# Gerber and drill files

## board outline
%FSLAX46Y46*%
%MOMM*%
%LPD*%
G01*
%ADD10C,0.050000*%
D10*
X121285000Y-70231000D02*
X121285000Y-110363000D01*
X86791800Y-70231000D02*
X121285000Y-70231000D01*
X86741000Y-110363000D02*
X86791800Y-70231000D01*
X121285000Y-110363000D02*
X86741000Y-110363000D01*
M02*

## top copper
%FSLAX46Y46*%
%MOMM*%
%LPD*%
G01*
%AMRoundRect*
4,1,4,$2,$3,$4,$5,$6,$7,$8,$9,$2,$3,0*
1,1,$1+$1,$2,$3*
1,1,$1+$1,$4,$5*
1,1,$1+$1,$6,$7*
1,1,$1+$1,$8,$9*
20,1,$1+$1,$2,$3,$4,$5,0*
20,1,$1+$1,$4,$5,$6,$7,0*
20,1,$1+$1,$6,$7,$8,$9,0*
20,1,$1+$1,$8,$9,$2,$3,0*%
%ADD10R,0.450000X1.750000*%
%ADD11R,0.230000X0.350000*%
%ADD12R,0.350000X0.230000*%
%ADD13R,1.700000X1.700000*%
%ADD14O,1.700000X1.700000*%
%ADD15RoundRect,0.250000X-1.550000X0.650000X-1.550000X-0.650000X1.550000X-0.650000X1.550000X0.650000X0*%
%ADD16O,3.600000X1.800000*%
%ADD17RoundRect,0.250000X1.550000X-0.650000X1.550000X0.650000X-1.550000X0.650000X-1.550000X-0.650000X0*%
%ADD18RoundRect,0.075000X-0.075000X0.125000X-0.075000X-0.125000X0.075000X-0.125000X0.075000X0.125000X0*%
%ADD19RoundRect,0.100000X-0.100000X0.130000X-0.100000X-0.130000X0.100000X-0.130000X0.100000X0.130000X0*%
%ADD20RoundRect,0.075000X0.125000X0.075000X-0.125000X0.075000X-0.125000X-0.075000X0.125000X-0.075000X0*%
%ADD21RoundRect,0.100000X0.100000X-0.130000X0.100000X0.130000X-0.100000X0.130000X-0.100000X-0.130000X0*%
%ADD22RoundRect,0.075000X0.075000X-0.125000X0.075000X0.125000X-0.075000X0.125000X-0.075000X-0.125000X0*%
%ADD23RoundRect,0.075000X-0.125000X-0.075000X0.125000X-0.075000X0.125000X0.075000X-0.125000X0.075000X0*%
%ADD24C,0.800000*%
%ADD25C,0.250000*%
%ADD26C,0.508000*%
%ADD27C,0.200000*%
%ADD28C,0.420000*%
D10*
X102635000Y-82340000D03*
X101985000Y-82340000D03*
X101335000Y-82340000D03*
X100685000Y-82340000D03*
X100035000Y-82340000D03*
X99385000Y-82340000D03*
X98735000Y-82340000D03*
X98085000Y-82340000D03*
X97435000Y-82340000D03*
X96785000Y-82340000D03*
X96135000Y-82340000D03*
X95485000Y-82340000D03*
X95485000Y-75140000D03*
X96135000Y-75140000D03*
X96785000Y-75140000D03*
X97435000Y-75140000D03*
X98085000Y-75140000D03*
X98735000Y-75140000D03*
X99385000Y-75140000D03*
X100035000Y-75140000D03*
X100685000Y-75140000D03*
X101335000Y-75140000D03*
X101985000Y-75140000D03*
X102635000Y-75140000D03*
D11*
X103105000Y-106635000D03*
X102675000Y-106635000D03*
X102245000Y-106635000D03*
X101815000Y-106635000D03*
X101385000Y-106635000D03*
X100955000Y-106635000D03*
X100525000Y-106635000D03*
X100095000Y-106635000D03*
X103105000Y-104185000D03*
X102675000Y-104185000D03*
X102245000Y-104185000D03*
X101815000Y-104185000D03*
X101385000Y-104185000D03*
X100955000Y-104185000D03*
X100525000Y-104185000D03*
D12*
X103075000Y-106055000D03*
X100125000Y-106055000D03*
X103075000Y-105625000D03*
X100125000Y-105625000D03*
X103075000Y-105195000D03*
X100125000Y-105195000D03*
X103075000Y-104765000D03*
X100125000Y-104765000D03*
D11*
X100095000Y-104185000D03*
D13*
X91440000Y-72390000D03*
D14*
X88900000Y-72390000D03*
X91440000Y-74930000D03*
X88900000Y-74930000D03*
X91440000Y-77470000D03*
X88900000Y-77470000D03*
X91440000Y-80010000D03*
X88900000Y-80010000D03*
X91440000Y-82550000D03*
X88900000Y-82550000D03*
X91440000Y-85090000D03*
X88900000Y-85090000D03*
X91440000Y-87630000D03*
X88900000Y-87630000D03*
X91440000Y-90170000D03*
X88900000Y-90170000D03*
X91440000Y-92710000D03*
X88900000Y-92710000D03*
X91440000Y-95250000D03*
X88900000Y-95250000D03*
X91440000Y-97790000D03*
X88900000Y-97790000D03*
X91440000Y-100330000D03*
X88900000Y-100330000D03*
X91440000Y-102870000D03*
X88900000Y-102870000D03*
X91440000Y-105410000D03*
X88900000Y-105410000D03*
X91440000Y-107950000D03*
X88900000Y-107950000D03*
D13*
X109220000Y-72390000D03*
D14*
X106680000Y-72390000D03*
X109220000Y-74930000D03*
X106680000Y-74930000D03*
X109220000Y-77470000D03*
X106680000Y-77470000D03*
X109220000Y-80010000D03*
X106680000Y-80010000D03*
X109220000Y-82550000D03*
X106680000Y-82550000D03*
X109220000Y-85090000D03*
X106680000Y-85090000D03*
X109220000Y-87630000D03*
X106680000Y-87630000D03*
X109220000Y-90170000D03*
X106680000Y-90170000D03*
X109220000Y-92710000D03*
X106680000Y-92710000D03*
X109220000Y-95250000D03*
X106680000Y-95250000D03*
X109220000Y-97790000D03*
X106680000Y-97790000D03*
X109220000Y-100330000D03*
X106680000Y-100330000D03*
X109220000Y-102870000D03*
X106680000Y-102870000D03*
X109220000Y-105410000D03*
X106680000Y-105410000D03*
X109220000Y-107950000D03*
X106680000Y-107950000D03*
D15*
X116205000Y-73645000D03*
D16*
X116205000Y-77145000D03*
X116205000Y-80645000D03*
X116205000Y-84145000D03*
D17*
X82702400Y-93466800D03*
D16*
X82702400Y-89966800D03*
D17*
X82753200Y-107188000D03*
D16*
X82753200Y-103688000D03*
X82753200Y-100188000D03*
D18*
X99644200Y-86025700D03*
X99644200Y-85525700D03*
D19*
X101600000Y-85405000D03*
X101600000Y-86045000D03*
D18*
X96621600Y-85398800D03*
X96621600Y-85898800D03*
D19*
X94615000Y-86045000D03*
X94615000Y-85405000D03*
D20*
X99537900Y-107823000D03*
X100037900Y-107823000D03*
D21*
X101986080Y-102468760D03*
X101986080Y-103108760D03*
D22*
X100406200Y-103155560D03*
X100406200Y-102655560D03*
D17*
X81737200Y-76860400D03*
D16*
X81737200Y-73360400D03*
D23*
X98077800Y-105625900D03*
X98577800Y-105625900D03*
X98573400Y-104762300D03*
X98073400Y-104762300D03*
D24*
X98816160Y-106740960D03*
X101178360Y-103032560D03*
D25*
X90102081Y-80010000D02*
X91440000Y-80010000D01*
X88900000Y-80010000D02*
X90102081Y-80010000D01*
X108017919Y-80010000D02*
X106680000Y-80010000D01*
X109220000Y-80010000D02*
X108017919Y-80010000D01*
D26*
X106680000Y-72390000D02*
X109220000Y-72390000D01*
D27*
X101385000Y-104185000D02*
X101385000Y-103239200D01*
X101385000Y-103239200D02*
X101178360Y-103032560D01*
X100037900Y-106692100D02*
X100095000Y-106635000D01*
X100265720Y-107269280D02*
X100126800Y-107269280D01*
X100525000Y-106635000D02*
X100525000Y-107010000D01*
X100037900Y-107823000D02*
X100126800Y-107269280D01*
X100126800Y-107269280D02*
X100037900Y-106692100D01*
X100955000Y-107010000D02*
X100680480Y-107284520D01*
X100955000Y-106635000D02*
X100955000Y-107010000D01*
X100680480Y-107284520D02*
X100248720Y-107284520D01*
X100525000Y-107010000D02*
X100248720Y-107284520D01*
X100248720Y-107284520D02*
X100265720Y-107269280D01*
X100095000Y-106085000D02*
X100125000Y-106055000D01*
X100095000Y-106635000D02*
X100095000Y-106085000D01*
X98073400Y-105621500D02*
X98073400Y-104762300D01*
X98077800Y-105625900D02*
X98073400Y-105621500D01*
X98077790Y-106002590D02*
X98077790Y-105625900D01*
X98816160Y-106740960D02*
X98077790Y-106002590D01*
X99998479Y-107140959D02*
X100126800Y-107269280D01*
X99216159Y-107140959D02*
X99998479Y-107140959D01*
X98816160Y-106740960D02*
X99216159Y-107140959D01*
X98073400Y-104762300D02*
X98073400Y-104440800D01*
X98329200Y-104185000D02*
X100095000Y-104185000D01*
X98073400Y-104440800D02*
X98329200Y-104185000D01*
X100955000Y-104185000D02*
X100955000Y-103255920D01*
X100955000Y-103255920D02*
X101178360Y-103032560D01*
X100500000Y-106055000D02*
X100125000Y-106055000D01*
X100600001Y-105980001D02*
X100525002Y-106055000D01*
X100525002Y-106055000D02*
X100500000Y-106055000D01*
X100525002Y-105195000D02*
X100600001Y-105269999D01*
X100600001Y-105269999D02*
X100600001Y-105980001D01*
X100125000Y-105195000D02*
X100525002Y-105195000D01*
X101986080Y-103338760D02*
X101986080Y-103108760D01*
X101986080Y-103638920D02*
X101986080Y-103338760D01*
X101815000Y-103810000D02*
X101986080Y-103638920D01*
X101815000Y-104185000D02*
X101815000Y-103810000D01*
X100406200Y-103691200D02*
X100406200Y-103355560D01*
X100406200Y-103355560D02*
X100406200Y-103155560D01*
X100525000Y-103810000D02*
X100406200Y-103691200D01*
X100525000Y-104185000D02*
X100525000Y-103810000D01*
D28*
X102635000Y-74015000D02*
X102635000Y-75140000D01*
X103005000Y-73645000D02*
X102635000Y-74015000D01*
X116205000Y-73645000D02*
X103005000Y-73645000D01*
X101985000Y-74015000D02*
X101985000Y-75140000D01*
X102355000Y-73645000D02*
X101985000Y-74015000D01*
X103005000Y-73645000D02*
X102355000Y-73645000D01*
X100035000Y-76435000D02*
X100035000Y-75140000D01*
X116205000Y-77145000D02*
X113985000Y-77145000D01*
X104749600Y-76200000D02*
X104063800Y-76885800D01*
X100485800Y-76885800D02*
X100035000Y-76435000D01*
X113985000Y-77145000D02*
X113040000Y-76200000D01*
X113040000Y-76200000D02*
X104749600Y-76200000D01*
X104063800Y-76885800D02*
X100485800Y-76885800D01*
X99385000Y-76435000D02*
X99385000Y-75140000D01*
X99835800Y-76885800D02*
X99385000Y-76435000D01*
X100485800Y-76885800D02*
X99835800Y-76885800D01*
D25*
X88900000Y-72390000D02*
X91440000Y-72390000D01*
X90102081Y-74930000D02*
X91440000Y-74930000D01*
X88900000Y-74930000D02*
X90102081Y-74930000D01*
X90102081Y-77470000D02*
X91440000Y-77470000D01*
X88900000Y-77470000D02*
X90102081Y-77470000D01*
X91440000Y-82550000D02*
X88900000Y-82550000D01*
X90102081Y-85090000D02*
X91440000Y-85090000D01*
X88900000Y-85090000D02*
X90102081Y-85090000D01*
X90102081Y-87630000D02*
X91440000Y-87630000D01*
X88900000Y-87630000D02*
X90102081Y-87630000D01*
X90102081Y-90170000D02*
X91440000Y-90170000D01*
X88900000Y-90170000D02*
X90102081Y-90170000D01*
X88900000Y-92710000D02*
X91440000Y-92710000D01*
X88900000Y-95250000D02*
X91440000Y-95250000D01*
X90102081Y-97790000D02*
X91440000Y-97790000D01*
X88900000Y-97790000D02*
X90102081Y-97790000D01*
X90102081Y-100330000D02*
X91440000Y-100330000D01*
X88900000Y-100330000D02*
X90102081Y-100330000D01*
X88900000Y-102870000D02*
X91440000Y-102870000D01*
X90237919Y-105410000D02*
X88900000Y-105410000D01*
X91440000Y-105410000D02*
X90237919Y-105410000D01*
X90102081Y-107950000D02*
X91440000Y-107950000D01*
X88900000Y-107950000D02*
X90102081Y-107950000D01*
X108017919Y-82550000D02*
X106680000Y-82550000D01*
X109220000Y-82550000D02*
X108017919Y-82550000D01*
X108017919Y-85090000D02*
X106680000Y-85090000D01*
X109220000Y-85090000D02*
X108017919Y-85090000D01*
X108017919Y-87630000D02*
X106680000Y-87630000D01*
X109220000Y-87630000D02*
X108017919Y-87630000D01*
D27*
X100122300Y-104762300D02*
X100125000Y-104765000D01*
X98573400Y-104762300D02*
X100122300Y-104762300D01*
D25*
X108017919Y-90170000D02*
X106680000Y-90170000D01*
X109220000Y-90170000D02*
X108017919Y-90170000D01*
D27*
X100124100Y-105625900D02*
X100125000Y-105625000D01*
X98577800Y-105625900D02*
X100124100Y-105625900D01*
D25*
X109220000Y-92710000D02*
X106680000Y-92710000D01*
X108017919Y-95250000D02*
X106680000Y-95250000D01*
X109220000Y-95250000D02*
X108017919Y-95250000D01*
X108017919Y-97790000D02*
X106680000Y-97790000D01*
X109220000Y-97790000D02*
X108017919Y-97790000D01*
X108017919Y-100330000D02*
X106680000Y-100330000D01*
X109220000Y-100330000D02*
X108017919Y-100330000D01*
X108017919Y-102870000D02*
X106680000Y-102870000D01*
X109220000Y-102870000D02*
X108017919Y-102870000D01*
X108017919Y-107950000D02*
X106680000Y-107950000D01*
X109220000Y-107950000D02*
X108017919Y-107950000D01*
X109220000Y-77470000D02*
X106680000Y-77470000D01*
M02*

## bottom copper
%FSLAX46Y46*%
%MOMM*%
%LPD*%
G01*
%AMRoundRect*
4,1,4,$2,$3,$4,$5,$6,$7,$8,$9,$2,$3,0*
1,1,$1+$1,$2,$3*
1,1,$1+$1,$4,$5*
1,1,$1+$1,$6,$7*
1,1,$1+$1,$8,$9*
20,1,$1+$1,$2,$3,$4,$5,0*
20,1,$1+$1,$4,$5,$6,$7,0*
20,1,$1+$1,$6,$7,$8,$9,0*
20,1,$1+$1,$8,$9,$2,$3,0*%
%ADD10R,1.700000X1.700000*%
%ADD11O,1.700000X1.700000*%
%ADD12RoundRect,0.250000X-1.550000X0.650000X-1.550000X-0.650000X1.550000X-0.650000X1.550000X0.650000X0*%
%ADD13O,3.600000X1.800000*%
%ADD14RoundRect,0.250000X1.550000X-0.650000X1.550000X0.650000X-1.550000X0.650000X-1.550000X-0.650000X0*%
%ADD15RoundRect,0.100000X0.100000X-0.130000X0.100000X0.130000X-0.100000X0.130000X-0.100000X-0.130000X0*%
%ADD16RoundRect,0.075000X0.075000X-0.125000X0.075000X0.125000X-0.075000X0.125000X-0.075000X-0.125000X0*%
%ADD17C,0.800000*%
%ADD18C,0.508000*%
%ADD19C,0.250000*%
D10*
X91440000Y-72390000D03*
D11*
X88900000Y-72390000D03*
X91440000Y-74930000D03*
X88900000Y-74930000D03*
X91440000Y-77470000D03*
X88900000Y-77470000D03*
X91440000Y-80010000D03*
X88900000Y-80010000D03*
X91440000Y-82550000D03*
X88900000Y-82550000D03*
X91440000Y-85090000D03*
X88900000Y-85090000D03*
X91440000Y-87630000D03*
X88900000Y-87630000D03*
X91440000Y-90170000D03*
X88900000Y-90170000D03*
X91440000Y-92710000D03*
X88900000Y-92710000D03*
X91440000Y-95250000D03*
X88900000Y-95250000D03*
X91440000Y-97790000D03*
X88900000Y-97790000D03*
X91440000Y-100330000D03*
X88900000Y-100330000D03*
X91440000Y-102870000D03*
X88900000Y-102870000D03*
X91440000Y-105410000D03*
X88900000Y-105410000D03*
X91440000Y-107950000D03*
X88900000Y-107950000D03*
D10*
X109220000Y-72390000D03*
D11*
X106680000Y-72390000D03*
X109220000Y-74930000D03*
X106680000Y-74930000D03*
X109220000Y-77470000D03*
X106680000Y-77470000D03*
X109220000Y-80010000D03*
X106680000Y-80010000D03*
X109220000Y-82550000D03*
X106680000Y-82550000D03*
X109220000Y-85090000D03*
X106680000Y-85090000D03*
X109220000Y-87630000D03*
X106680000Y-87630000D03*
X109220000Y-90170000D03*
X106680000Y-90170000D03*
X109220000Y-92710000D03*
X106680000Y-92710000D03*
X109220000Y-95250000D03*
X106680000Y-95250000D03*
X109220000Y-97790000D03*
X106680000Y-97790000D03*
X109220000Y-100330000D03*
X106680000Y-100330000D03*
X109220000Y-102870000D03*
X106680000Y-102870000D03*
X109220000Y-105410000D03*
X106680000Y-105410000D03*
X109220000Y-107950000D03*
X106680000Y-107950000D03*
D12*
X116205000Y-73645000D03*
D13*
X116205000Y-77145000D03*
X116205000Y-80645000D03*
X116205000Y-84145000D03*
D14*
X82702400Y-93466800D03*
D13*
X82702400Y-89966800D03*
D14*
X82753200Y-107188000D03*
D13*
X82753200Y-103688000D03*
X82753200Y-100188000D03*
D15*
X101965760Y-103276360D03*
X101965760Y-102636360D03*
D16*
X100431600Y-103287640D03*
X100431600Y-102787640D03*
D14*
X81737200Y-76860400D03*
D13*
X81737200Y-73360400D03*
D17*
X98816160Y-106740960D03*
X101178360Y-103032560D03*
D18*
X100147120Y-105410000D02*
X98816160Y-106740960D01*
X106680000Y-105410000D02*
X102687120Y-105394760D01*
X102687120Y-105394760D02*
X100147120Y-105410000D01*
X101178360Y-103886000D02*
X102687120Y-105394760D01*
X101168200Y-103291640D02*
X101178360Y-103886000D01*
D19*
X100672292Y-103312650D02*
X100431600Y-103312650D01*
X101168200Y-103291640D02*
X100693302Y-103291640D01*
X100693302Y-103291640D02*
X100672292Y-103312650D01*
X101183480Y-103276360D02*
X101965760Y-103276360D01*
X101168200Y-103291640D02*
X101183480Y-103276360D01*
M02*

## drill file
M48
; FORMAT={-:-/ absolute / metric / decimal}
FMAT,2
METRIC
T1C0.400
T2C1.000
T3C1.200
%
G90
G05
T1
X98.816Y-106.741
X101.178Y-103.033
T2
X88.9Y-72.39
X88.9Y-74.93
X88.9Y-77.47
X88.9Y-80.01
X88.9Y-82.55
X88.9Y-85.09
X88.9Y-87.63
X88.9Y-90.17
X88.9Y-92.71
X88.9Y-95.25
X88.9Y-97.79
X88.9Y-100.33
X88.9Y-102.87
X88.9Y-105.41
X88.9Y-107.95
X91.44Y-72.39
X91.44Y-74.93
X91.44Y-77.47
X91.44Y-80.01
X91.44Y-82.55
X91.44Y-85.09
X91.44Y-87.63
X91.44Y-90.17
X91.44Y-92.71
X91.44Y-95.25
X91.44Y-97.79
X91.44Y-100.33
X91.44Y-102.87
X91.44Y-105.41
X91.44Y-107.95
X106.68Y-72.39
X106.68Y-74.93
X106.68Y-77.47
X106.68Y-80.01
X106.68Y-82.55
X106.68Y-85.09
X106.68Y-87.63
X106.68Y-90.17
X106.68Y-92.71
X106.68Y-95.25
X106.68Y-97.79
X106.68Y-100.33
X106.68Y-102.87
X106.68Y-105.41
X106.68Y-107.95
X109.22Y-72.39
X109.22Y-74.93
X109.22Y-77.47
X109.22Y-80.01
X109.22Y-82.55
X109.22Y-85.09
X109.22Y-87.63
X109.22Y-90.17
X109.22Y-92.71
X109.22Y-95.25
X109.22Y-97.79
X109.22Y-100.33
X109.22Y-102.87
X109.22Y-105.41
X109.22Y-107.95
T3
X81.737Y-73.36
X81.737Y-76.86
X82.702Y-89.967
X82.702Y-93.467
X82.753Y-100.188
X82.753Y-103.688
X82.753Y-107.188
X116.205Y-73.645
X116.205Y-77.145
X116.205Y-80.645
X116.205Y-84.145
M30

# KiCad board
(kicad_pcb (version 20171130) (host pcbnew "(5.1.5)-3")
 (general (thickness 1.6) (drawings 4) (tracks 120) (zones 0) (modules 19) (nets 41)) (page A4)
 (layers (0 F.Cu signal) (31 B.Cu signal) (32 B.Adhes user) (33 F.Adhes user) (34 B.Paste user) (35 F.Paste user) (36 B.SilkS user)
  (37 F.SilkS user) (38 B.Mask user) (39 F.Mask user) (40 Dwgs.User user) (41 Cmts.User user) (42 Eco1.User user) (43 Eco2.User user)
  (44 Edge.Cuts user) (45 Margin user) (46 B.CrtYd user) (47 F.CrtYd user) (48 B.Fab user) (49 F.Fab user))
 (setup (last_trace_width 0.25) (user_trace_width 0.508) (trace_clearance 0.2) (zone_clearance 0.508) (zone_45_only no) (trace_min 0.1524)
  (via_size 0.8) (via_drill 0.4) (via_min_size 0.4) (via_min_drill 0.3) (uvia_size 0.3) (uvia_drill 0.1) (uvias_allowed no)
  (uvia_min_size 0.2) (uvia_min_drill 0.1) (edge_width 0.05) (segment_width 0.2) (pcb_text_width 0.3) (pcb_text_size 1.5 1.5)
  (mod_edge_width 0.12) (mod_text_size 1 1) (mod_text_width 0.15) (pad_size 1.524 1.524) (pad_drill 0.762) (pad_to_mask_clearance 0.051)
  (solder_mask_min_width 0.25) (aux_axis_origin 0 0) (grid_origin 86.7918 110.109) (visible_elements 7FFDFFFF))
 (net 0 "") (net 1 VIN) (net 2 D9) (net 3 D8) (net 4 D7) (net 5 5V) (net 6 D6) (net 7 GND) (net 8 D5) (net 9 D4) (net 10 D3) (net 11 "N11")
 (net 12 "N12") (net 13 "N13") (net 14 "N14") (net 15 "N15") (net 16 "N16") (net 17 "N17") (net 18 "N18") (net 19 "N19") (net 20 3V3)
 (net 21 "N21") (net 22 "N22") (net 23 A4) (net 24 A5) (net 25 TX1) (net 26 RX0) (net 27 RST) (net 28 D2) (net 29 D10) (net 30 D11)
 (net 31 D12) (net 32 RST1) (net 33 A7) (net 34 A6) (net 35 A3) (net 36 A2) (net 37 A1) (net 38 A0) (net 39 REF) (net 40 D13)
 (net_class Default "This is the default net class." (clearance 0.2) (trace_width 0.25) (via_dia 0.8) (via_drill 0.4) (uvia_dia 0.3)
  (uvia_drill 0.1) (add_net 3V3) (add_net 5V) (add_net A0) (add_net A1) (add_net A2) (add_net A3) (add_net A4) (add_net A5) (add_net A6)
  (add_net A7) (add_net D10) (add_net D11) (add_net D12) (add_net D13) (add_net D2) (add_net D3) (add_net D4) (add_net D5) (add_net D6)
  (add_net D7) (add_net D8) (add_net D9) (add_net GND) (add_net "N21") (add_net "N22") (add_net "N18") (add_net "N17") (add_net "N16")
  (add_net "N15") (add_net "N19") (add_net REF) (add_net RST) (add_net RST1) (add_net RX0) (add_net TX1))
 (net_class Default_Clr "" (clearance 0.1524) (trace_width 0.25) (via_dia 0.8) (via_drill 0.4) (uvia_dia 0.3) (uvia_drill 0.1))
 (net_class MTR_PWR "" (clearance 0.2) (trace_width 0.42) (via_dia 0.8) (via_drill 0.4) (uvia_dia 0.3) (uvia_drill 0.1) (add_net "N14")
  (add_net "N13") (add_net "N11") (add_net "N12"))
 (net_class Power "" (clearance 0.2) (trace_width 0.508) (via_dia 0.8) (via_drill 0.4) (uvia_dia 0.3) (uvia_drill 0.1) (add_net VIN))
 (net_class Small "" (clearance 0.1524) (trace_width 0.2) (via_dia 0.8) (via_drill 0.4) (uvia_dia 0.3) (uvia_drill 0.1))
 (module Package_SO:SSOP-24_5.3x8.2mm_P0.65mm (layer F.Cu) (at 99.06 78.74 270)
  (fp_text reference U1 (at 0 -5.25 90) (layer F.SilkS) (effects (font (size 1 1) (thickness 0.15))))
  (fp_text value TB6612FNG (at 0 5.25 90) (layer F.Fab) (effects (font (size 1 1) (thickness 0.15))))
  (pad 24 smd rect (at 3.6 -3.575 270) (size 1.75 0.45) (layers F.Cu F.Paste F.Mask) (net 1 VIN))
  (pad 23 smd rect (at 3.6 -2.925 270) (size 1.75 0.45) (layers F.Cu F.Paste F.Mask) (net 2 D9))
  (pad 22 smd rect (at 3.6 -2.275 270) (size 1.75 0.45) (layers F.Cu F.Paste F.Mask) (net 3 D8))
  (pad 21 smd rect (at 3.6 -1.625 270) (size 1.75 0.45) (layers F.Cu F.Paste F.Mask) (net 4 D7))
  (pad 20 smd rect (at 3.6 -0.975 270) (size 1.75 0.45) (layers F.Cu F.Paste F.Mask) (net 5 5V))
  (pad 19 smd rect (at 3.6 -0.325 270) (size 1.75 0.45) (layers F.Cu F.Paste F.Mask) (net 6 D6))
  (pad 18 smd rect (at 3.6 0.325 270) (size 1.75 0.45) (layers F.Cu F.Paste F.Mask) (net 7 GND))
  (pad 17 smd rect (at 3.6 0.975 270) (size 1.75 0.45) (layers F.Cu F.Paste F.Mask) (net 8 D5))
  (pad 16 smd rect (at 3.6 1.625 270) (size 1.75 0.45) (layers F.Cu F.Paste F.Mask) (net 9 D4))
  (pad 15 smd rect (at 3.6 2.275 270) (size 1.75 0.45) (layers F.Cu F.Paste F.Mask) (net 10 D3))
  (pad 14 smd rect (at 3.6 2.925 270) (size 1.75 0.45) (layers F.Cu F.Paste F.Mask) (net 1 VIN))
  (pad 13 smd rect (at 3.6 3.575 270) (size 1.75 0.45) (layers F.Cu F.Paste F.Mask) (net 1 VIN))
  (pad 12 smd rect (at -3.6 3.575 270) (size 1.75 0.45) (layers F.Cu F.Paste F.Mask) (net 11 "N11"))
  (pad 11 smd rect (at -3.6 2.925 270) (size 1.75 0.45) (layers F.Cu F.Paste F.Mask) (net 11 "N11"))
  (pad 10 smd rect (at -3.6 2.275 270) (size 1.75 0.45) (layers F.Cu F.Paste F.Mask) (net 7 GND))
  (pad 9 smd rect (at -3.6 1.625 270) (size 1.75 0.45) (layers F.Cu F.Paste F.Mask) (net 7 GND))
  (pad 8 smd rect (at -3.6 0.975 270) (size 1.75 0.45) (layers F.Cu F.Paste F.Mask) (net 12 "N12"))
  (pad 7 smd rect (at -3.6 0.325 270) (size 1.75 0.45) (layers F.Cu F.Paste F.Mask) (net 12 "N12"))
  (pad 6 smd rect (at -3.6 -0.325 270) (size 1.75 0.45) (layers F.Cu F.Paste F.Mask) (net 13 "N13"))
  (pad 5 smd rect (at -3.6 -0.975 270) (size 1.75 0.45) (layers F.Cu F.Paste F.Mask) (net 13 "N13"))
  (pad 4 smd rect (at -3.6 -1.625 270) (size 1.75 0.45) (layers F.Cu F.Paste F.Mask) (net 7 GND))
  (pad 3 smd rect (at -3.6 -2.275 270) (size 1.75 0.45) (layers F.Cu F.Paste F.Mask) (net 7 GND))
  (pad 2 smd rect (at -3.6 -2.925 270) (size 1.75 0.45) (layers F.Cu F.Paste F.Mask) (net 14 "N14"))
  (pad 1 smd rect (at -3.6 -3.575 270) (size 1.75 0.45) (layers F.Cu F.Paste F.Mask) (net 14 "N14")))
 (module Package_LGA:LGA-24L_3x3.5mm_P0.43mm (layer F.Cu) (at 101.6 105.41)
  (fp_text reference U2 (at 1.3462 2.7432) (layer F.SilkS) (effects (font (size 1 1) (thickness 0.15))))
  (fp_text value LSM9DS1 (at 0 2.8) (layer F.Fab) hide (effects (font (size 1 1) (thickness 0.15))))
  (pad 13 smd rect (at 1.505 1.225) (size 0.23 0.35) (layers F.Cu F.Paste F.Mask) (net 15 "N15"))
  (pad 12 smd rect (at 1.075 1.225) (size 0.23 0.35) (layers F.Cu F.Paste F.Mask) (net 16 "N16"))
  (pad 11 smd rect (at 0.645 1.225) (size 0.23 0.35) (layers F.Cu F.Paste F.Mask) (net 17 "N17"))
  (pad 10 smd rect (at 0.215 1.225) (size 0.23 0.35) (layers F.Cu F.Paste F.Mask) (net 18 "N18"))
  (pad 9 smd rect (at -0.215 1.225) (size 0.23 0.35) (layers F.Cu F.Paste F.Mask) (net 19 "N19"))
  (pad 8 smd rect (at -0.645 1.225) (size 0.23 0.35) (layers F.Cu F.Paste F.Mask) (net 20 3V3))
  (pad 7 smd rect (at -1.075 1.225) (size 0.23 0.35) (layers F.Cu F.Paste F.Mask) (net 20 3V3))
  (pad 6 smd rect (at -1.505 1.225) (size 0.23 0.35) (layers F.Cu F.Paste F.Mask) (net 20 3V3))
  (pad 18 smd rect (at 1.505 -1.225) (size 0.23 0.35) (layers F.Cu F.Paste F.Mask) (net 7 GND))
  (pad 19 smd rect (at 1.075 -1.225) (size 0.23 0.35) (layers F.Cu F.Paste F.Mask) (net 7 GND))
  (pad 20 smd rect (at 0.645 -1.225) (size 0.23 0.35) (layers F.Cu F.Paste F.Mask) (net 7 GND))
  (pad 21 smd rect (at 0.215 -1.225) (size 0.23 0.35) (layers F.Cu F.Paste F.Mask) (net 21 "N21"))
  (pad 22 smd rect (at -0.215 -1.225) (size 0.23 0.35) (layers F.Cu F.Paste F.Mask) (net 20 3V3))
  (pad 23 smd rect (at -0.645 -1.225) (size 0.23 0.35) (layers F.Cu F.Paste F.Mask) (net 20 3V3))
  (pad 24 smd rect (at -1.075 -1.225) (size 0.23 0.35) (layers F.Cu F.Paste F.Mask) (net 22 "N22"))
  (pad 14 smd rect (at 1.475 0.645) (size 0.35 0.23) (layers F.Cu F.Paste F.Mask) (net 7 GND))
  (pad 5 smd rect (at -1.475 0.645) (size 0.35 0.23) (layers F.Cu F.Paste F.Mask) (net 20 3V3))
  (pad 15 smd rect (at 1.475 0.215) (size 0.35 0.23) (layers F.Cu F.Paste F.Mask) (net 7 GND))
  (pad 4 smd rect (at -1.475 0.215) (size 0.35 0.23) (layers F.Cu F.Paste F.Mask) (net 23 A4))
  (pad 16 smd rect (at 1.475 -0.215) (size 0.35 0.23) (layers F.Cu F.Paste F.Mask) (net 7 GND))
  (pad 3 smd rect (at -1.475 -0.215) (size 0.35 0.23) (layers F.Cu F.Paste F.Mask) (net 20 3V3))
  (pad 17 smd rect (at 1.475 -0.645) (size 0.35 0.23) (layers F.Cu F.Paste F.Mask) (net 7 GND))
  (pad 2 smd rect (at -1.475 -0.645) (size 0.35 0.23) (layers F.Cu F.Paste F.Mask) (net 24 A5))
  (pad 1 smd rect (at -1.505 -1.225) (size 0.23 0.35) (layers F.Cu F.Paste F.Mask) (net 20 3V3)))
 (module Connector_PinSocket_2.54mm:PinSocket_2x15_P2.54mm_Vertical (layer F.Cu) (at 91.44 72.39)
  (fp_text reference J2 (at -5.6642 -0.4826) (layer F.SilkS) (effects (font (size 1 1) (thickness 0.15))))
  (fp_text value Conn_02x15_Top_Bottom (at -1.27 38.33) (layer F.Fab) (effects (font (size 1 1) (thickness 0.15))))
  (pad 1 thru_hole rect (at 0 0) (size 1.7 1.7) (drill 1) (layers *.Cu *.Mask) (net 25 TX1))
  (pad 2 thru_hole oval (at -2.54 0) (size 1.7 1.7) (drill 1) (layers *.Cu *.Mask) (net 25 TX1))
  (pad 3 thru_hole oval (at 0 2.54) (size 1.7 1.7) (drill 1) (layers *.Cu *.Mask) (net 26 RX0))
  (pad 4 thru_hole oval (at -2.54 2.54) (size 1.7 1.7) (drill 1) (layers *.Cu *.Mask) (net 26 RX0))
  (pad 5 thru_hole oval (at 0 5.08) (size 1.7 1.7) (drill 1) (layers *.Cu *.Mask) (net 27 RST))
  (pad 6 thru_hole oval (at -2.54 5.08) (size 1.7 1.7) (drill 1) (layers *.Cu *.Mask) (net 27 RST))
  (pad 7 thru_hole oval (at 0 7.62) (size 1.7 1.7) (drill 1) (layers *.Cu *.Mask) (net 7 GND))
  (pad 8 thru_hole oval (at -2.54 7.62) (size 1.7 1.7) (drill 1) (layers *.Cu *.Mask) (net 7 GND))
  (pad 9 thru_hole oval (at 0 10.16) (size 1.7 1.7) (drill 1) (layers *.Cu *.Mask) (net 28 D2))
  (pad 10 thru_hole oval (at -2.54 10.16) (size 1.7 1.7) (drill 1) (layers *.Cu *.Mask) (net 28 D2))
  (pad 11 thru_hole oval (at 0 12.7) (size 1.7 1.7) (drill 1) (layers *.Cu *.Mask) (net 10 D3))
  (pad 12 thru_hole oval (at -2.54 12.7) (size 1.7 1.7) (drill 1) (layers *.Cu *.Mask) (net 10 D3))
  (pad 13 thru_hole oval (at 0 15.24) (size 1.7 1.7) (drill 1) (layers *.Cu *.Mask) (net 9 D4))
  (pad 14 thru_hole oval (at -2.54 15.24) (size 1.7 1.7) (drill 1) (layers *.Cu *.Mask) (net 9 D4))
  (pad 15 thru_hole oval (at 0 17.78) (size 1.7 1.7) (drill 1) (layers *.Cu *.Mask) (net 8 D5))
  (pad 16 thru_hole oval (at -2.54 17.78) (size 1.7 1.7) (drill 1) (layers *.Cu *.Mask) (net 8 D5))
  (pad 17 thru_hole oval (at 0 20.32) (size 1.7 1.7) (drill 1) (layers *.Cu *.Mask) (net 6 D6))
  (pad 18 thru_hole oval (at -2.54 20.32) (size 1.7 1.7) (drill 1) (layers *.Cu *.Mask) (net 6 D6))
  (pad 19 thru_hole oval (at 0 22.86) (size 1.7 1.7) (drill 1) (layers *.Cu *.Mask) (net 4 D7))
  (pad 20 thru_hole oval (at -2.54 22.86) (size 1.7 1.7) (drill 1) (layers *.Cu *.Mask) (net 4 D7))
  (pad 21 thru_hole oval (at 0 25.4) (size 1.7 1.7) (drill 1) (layers *.Cu *.Mask) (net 3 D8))
  (pad 22 thru_hole oval (at -2.54 25.4) (size 1.7 1.7) (drill 1) (layers *.Cu *.Mask) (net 3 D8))
  (pad 23 thru_hole oval (at 0 27.94) (size 1.7 1.7) (drill 1) (layers *.Cu *.Mask) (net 2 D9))
  (pad 24 thru_hole oval (at -2.54 27.94) (size 1.7 1.7) (drill 1) (layers *.Cu *.Mask) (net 2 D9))
  (pad 25 thru_hole oval (at 0 30.48) (size 1.7 1.7) (drill 1) (layers *.Cu *.Mask) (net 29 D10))
  (pad 26 thru_hole oval (at -2.54 30.48) (size 1.7 1.7) (drill 1) (layers *.Cu *.Mask) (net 29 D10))
  (pad 27 thru_hole oval (at 0 33.02) (size 1.7 1.7) (drill 1) (layers *.Cu *.Mask) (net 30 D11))
  (pad 28 thru_hole oval (at -2.54 33.02) (size 1.7 1.7) (drill 1) (layers *.Cu *.Mask) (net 30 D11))
  (pad 29 thru_hole oval (at 0 35.56) (size 1.7 1.7) (drill 1) (layers *.Cu *.Mask) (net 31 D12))
  (pad 30 thru_hole oval (at -2.54 35.56) (size 1.7 1.7) (drill 1) (layers *.Cu *.Mask) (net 31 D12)))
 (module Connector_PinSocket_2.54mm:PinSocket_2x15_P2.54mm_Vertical (layer F.Cu) (at 109.22 72.39)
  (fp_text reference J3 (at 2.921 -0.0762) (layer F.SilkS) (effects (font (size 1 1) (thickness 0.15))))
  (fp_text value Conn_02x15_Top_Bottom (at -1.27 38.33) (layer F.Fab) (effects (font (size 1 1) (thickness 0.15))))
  (pad 1 thru_hole rect (at 0 0) (size 1.7 1.7) (drill 1) (layers *.Cu *.Mask) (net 1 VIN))
  (pad 2 thru_hole oval (at -2.54 0) (size 1.7 1.7) (drill 1) (layers *.Cu *.Mask) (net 1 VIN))
  (pad 3 thru_hole oval (at 0 2.54) (size 1.7 1.7) (drill 1) (layers *.Cu *.Mask) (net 7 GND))
  (pad 4 thru_hole oval (at -2.54 2.54) (size 1.7 1.7) (drill 1) (layers *.Cu *.Mask) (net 7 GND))
  (pad 5 thru_hole oval (at 0 5.08) (size 1.7 1.7) (drill 1) (layers *.Cu *.Mask) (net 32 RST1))
  (pad 6 thru_hole oval (at -2.54 5.08) (size 1.7 1.7) (drill 1) (layers *.Cu *.Mask) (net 32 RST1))
  (pad 7 thru_hole oval (at 0 7.62) (size 1.7 1.7) (drill 1) (layers *.Cu *.Mask) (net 5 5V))
  (pad 8 thru_hole oval (at -2.54 7.62) (size 1.7 1.7) (drill 1) (layers *.Cu *.Mask) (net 5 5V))
  (pad 9 thru_hole oval (at 0 10.16) (size 1.7 1.7) (drill 1) (layers *.Cu *.Mask) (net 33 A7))
  (pad 10 thru_hole oval (at -2.54 10.16) (size 1.7 1.7) (drill 1) (layers *.Cu *.Mask) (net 33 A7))
  (pad 11 thru_hole oval (at 0 12.7) (size 1.7 1.7) (drill 1) (layers *.Cu *.Mask) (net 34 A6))
  (pad 12 thru_hole oval (at -2.54 12.7) (size 1.7 1.7) (drill 1) (layers *.Cu *.Mask) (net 34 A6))
  (pad 13 thru_hole oval (at 0 15.24) (size 1.7 1.7) (drill 1) (layers *.Cu *.Mask) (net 24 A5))
  (pad 14 thru_hole oval (at -2.54 15.24) (size 1.7 1.7) (drill 1) (layers *.Cu *.Mask) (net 24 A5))
  (pad 15 thru_hole oval (at 0 17.78) (size 1.7 1.7) (drill 1) (layers *.Cu *.Mask) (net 23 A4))
  (pad 16 thru_hole oval (at -2.54 17.78) (size 1.7 1.7) (drill 1) (layers *.Cu *.Mask) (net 23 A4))
  (pad 17 thru_hole oval (at 0 20.32) (size 1.7 1.7) (drill 1) (layers *.Cu *.Mask) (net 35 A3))
  (pad 18 thru_hole oval (at -2.54 20.32) (size 1.7 1.7) (drill 1) (layers *.Cu *.Mask) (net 35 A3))
  (pad 19 thru_hole oval (at 0 22.86) (size 1.7 1.7) (drill 1) (layers *.Cu *.Mask) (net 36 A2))
  (pad 20 thru_hole oval (at -2.54 22.86) (size 1.7 1.7) (drill 1) (layers *.Cu *.Mask) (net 36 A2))
  (pad 21 thru_hole oval (at 0 25.4) (size 1.7 1.7) (drill 1) (layers *.Cu *.Mask) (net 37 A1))
  (pad 22 thru_hole oval (at -2.54 25.4) (size 1.7 1.7) (drill 1) (layers *.Cu *.Mask) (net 37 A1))
  (pad 23 thru_hole oval (at 0 27.94) (size 1.7 1.7) (drill 1) (layers *.Cu *.Mask) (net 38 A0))
  (pad 24 thru_hole oval (at -2.54 27.94) (size 1.7 1.7) (drill 1) (layers *.Cu *.Mask) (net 38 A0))
  (pad 25 thru_hole oval (at 0 30.48) (size 1.7 1.7) (drill 1) (layers *.Cu *.Mask) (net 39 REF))
  (pad 26 thru_hole oval (at -2.54 30.48) (size 1.7 1.7) (drill 1) (layers *.Cu *.Mask) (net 39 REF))
  (pad 27 thru_hole oval (at 0 33.02) (size 1.7 1.7) (drill 1) (layers *.Cu *.Mask) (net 20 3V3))
  (pad 28 thru_hole oval (at -2.54 33.02) (size 1.7 1.7) (drill 1) (layers *.Cu *.Mask) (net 20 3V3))
  (pad 29 thru_hole oval (at 0 35.56) (size 1.7 1.7) (drill 1) (layers *.Cu *.Mask) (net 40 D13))
  (pad 30 thru_hole oval (at -2.54 35.56) (size 1.7 1.7) (drill 1) (layers *.Cu *.Mask) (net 40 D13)))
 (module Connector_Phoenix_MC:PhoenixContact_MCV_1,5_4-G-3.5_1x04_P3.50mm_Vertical (layer F.Cu) (at 116.205 73.645 270)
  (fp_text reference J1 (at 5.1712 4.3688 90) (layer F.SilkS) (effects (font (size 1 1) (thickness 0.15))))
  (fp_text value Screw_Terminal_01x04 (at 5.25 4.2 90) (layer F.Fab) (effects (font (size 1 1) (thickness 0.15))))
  (pad 1 thru_hole roundrect (at 0 0 270) (size 1.8 3.6) (drill 1.2) (layers *.Cu *.Mask) (roundrect_rratio 0.138889) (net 14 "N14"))
  (pad 2 thru_hole oval (at 3.5 0 270) (size 1.8 3.6) (drill 1.2) (layers *.Cu *.Mask) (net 13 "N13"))
  (pad 3 thru_hole oval (at 7 0 270) (size 1.8 3.6) (drill 1.2) (layers *.Cu *.Mask) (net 11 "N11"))
  (pad 4 thru_hole oval (at 10.5 0 270) (size 1.8 3.6) (drill 1.2) (layers *.Cu *.Mask) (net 12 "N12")))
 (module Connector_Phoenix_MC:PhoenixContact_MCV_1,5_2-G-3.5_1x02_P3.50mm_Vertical (layer F.Cu) (at 82.7024 93.4668 90)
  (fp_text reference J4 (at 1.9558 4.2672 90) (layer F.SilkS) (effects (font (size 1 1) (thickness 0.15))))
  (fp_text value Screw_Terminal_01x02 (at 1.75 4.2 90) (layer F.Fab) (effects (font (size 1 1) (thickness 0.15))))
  (pad 1 thru_hole roundrect (at 0 0 90) (size 1.8 3.6) (drill 1.2) (layers *.Cu *.Mask) (roundrect_rratio 0.138889) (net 1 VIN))
  (pad 2 thru_hole oval (at 3.5 0 90) (size 1.8 3.6) (drill 1.2) (layers *.Cu *.Mask) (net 7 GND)))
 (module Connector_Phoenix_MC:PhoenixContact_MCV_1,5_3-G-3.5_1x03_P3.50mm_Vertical (layer F.Cu) (at 82.7532 107.188 90)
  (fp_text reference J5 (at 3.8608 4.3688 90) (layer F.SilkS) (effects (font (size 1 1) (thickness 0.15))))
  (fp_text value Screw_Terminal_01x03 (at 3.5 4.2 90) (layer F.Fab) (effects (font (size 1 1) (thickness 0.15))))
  (pad 1 thru_hole roundrect (at 0 0 90) (size 1.8 3.6) (drill 1.2) (layers *.Cu *.Mask) (roundrect_rratio 0.138889) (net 29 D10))
  (pad 2 thru_hole oval (at 3.5 0 90) (size 1.8 3.6) (drill 1.2) (layers *.Cu *.Mask) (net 30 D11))
  (pad 3 thru_hole oval (at 7 0 90) (size 1.8 3.6) (drill 1.2) (layers *.Cu *.Mask) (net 31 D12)))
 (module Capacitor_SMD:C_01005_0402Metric (layer F.Cu) (at 99.6442 85.7757 270)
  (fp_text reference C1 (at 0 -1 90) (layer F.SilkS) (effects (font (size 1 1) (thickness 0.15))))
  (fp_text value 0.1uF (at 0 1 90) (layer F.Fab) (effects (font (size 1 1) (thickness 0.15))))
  (pad 2 smd roundrect (at 0.25 0 270) (size 0.4 0.3) (layers F.Cu F.Mask) (roundrect_rratio 0.25) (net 7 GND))
  (pad 1 smd roundrect (at -0.25 0 270) (size 0.4 0.3) (layers F.Cu F.Mask) (roundrect_rratio 0.25) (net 5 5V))
  (pad "" smd roundrect (at 0.275 0 270) (size 0.27 0.27) (layers F.Paste) (roundrect_rratio 0.25))
  (pad "" smd roundrect (at -0.275 0 270) (size 0.27 0.27) (layers F.Paste) (roundrect_rratio 0.25)))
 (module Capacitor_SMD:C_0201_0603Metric (layer F.Cu) (at 101.6 85.725 270)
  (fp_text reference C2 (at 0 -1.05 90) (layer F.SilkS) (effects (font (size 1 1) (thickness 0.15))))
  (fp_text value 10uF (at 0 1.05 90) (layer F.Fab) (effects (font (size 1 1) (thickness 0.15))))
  (pad "" smd roundrect (at -0.345 0 270) (size 0.318 0.36) (layers F.Paste) (roundrect_rratio 0.25))
  (pad "" smd roundrect (at 0.345 0 270) (size 0.318 0.36) (layers F.Paste) (roundrect_rratio 0.25))
  (pad 1 smd roundrect (at -0.32 0 270) (size 0.46 0.4) (layers F.Cu F.Mask) (roundrect_rratio 0.25) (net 5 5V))
  (pad 2 smd roundrect (at 0.32 0 270) (size 0.46 0.4) (layers F.Cu F.Mask) (roundrect_rratio 0.25) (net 7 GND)))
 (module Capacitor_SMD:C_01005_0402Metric (layer F.Cu) (at 96.6216 85.6488 270)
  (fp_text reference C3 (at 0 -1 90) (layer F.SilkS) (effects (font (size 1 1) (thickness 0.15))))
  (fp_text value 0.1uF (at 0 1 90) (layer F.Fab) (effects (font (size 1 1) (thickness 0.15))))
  (pad "" smd roundrect (at -0.275 0 270) (size 0.27 0.27) (layers F.Paste) (roundrect_rratio 0.25))
  (pad "" smd roundrect (at 0.275 0 270) (size 0.27 0.27) (layers F.Paste) (roundrect_rratio 0.25))
  (pad 1 smd roundrect (at -0.25 0 270) (size 0.4 0.3) (layers F.Cu F.Mask) (roundrect_rratio 0.25) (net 1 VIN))
  (pad 2 smd roundrect (at 0.25 0 270) (size 0.4 0.3) (layers F.Cu F.Mask) (roundrect_rratio 0.25) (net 7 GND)))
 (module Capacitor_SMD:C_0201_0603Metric (layer F.Cu) (at 94.615 85.725 270)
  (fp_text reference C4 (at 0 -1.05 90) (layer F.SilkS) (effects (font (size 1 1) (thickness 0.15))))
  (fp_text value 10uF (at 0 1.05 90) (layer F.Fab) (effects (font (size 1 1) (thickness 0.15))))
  (pad 2 smd roundrect (at 0.32 0 270) (size 0.46 0.4) (layers F.Cu F.Mask) (roundrect_rratio 0.25) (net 7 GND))
  (pad 1 smd roundrect (at -0.32 0 270) (size 0.46 0.4) (layers F.Cu F.Mask) (roundrect_rratio 0.25) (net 1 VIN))
  (pad "" smd roundrect (at 0.345 0 270) (size 0.318 0.36) (layers F.Paste) (roundrect_rratio 0.25))
  (pad "" smd roundrect (at -0.345 0 270) (size 0.318 0.36) (layers F.Paste) (roundrect_rratio 0.25)))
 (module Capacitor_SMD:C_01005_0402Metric (layer F.Cu) (at 99.7879 107.823 180)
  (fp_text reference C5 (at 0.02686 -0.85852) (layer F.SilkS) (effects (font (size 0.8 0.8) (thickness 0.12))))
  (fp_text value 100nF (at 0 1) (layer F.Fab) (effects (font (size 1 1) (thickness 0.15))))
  (pad 2 smd roundrect (at 0.25 0 180) (size 0.4 0.3) (layers F.Cu F.Mask) (roundrect_rratio 0.25) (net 7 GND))
  (pad 1 smd roundrect (at -0.25 0 180) (size 0.4 0.3) (layers F.Cu F.Mask) (roundrect_rratio 0.25) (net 20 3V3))
  (pad "" smd roundrect (at 0.275 0 180) (size 0.27 0.27) (layers F.Paste) (roundrect_rratio 0.25))
  (pad "" smd roundrect (at -0.275 0 180) (size 0.27 0.27) (layers F.Paste) (roundrect_rratio 0.25)))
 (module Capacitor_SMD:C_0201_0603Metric (layer B.Cu) (at 101.96576 102.95636 90)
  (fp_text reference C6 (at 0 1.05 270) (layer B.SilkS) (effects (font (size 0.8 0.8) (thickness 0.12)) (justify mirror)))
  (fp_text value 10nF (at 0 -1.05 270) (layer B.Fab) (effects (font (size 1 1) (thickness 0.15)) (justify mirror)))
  (pad "" smd roundrect (at -0.345 0 90) (size 0.318 0.36) (layers B.Paste) (roundrect_rratio 0.25))
  (pad "" smd roundrect (at 0.345 0 90) (size 0.318 0.36) (layers B.Paste) (roundrect_rratio 0.25))
  (pad 1 smd roundrect (at -0.32 0 90) (size 0.46 0.4) (layers B.Cu B.Mask) (roundrect_rratio 0.25) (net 20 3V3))
  (pad 2 smd roundrect (at 0.32 0 90) (size 0.46 0.4) (layers B.Cu B.Mask) (roundrect_rratio 0.25) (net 7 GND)))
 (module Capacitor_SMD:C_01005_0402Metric (layer B.Cu) (at 100.4316 103.03764 90)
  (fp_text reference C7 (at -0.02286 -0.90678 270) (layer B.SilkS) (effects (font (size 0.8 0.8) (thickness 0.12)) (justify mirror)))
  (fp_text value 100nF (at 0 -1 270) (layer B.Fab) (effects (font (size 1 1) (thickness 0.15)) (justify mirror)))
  (pad "" smd roundrect (at -0.275 0 90) (size 0.27 0.27) (layers B.Paste) (roundrect_rratio 0.25))
  (pad "" smd roundrect (at 0.275 0 90) (size 0.27 0.27) (layers B.Paste) (roundrect_rratio 0.25))
  (pad 1 smd roundrect (at -0.25 0 90) (size 0.4 0.3) (layers B.Cu B.Mask) (roundrect_rratio 0.25) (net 20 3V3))
  (pad 2 smd roundrect (at 0.25 0 90) (size 0.4 0.3) (layers B.Cu B.Mask) (roundrect_rratio 0.25) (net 7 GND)))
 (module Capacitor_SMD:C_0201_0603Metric (layer F.Cu) (at 101.98608 102.78876 90)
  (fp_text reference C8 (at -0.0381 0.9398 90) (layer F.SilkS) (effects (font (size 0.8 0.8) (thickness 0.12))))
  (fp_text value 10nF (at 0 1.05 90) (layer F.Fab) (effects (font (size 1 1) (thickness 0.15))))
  (pad 2 smd roundrect (at 0.32 0 90) (size 0.46 0.4) (layers F.Cu F.Mask) (roundrect_rratio 0.25) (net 7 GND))
  (pad 1 smd roundrect (at -0.32 0 90) (size 0.46 0.4) (layers F.Cu F.Mask) (roundrect_rratio 0.25) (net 21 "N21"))
  (pad "" smd roundrect (at 0.345 0 90) (size 0.318 0.36) (layers F.Paste) (roundrect_rratio 0.25))
  (pad "" smd roundrect (at -0.345 0 90) (size 0.318 0.36) (layers F.Paste) (roundrect_rratio 0.25)))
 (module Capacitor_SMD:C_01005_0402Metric (layer F.Cu) (at 100.4062 102.90556 90)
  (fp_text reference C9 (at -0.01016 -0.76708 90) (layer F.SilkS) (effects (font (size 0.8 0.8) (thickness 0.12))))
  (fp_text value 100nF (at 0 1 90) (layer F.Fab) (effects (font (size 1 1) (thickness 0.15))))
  (pad "" smd roundrect (at -0.275 0 90) (size 0.27 0.27) (layers F.Paste) (roundrect_rratio 0.25))
  (pad "" smd roundrect (at 0.275 0 90) (size 0.27 0.27) (layers F.Paste) (roundrect_rratio 0.25))
  (pad 1 smd roundrect (at -0.25 0 90) (size 0.4 0.3) (layers F.Cu F.Mask) (roundrect_rratio 0.25) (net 22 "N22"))
  (pad 2 smd roundrect (at 0.25 0 90) (size 0.4 0.3) (layers F.Cu F.Mask) (roundrect_rratio 0.25) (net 7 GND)))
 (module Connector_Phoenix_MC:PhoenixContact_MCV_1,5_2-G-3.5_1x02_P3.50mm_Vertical (layer F.Cu) (at 81.7372 76.8604 90)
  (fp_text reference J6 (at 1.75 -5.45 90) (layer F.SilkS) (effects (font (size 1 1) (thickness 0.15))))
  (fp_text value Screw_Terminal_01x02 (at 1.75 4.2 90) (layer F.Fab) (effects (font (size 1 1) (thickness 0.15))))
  (pad 1 thru_hole roundrect (at 0 0 90) (size 1.8 3.6) (drill 1.2) (layers *.Cu *.Mask) (roundrect_rratio 0.138889) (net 5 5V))
  (pad 2 thru_hole oval (at 3.5 0 90) (size 1.8 3.6) (drill 1.2) (layers *.Cu *.Mask) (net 7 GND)))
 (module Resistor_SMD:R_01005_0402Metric (layer F.Cu) (at 98.3278 105.6259)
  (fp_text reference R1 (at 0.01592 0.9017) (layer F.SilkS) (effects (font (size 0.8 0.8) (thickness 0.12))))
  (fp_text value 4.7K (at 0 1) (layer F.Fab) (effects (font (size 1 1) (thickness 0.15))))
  (pad "" smd roundrect (at -0.275 0) (size 0.27 0.27) (layers F.Paste) (roundrect_rratio 0.25))
  (pad "" smd roundrect (at 0.275 0) (size 0.27 0.27) (layers F.Paste) (roundrect_rratio 0.25))
  (pad 1 smd roundrect (at -0.25 0) (size 0.4 0.3) (layers F.Cu F.Mask) (roundrect_rratio 0.25) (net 20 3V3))
  (pad 2 smd roundrect (at 0.25 0) (size 0.4 0.3) (layers F.Cu F.Mask) (roundrect_rratio 0.25) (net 23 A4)))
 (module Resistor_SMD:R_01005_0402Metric (layer F.Cu) (at 98.3234 104.7623)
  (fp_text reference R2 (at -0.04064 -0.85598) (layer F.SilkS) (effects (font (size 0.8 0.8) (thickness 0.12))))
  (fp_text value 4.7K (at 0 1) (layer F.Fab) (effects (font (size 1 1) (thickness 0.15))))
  (pad 2 smd roundrect (at 0.25 0) (size 0.4 0.3) (layers F.Cu F.Mask) (roundrect_rratio 0.25) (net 24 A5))
  (pad 1 smd roundrect (at -0.25 0) (size 0.4 0.3) (layers F.Cu F.Mask) (roundrect_rratio 0.25) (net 20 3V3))
  (pad "" smd roundrect (at 0.275 0) (size 0.27 0.27) (layers F.Paste) (roundrect_rratio 0.25))
  (pad "" smd roundrect (at -0.275 0) (size 0.27 0.27) (layers F.Paste) (roundrect_rratio 0.25)))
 (gr_line (start 121.285 70.231) (end 121.285 110.363) (layer Edge.Cuts) (width 0.05))
 (gr_line (start 86.7918 70.231) (end 121.285 70.231) (layer Edge.Cuts) (width 0.05))
 (gr_line (start 86.741 110.363) (end 86.7918 70.231) (layer Edge.Cuts) (width 0.05))
 (gr_line (start 121.285 110.363) (end 86.741 110.363) (layer Edge.Cuts) (width 0.05))
 (segment (start 90.102081 80.01) (end 91.44 80.01) (width 0.25) (layer F.Cu) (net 7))
 (segment (start 88.9 80.01) (end 90.102081 80.01) (width 0.25) (layer F.Cu) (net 7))
 (segment (start 108.017919 80.01) (end 106.68 80.01) (width 0.25) (layer F.Cu) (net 5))
 (segment (start 109.22 80.01) (end 108.017919 80.01) (width 0.25) (layer F.Cu) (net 5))
 (segment (start 106.68 72.39) (end 109.22 72.39) (width 0.508) (layer F.Cu) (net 1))
 (segment (start 101.385 104.185) (end 101.385 103.2392) (width 0.2) (layer F.Cu) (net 20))
 (segment (start 101.385 103.2392) (end 101.17836 103.03256) (width 0.2) (layer F.Cu) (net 20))
 (segment (start 100.0379 106.6921) (end 100.095 106.635) (width 0.2) (layer F.Cu) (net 20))
 (segment (start 100.26572 107.26928) (end 100.1268 107.26928) (width 0.2) (layer F.Cu) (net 20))
 (segment (start 100.525 106.635) (end 100.525 107.01) (width 0.2) (layer F.Cu) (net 20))
 (segment (start 100.0379 107.823) (end 100.1268 107.26928) (width 0.2) (layer F.Cu) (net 20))
 (segment (start 100.1268 107.26928) (end 100.0379 106.6921) (width 0.2) (layer F.Cu) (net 20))
 (segment (start 100.955 107.01) (end 100.68048 107.28452) (width 0.2) (layer F.Cu) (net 20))
 (segment (start 100.955 106.635) (end 100.955 107.01) (width 0.2) (layer F.Cu) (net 20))
 (segment (start 100.68048 107.28452) (end 100.24872 107.28452) (width 0.2) (layer F.Cu) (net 20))
 (segment (start 100.525 107.01) (end 100.24872 107.28452) (width 0.2) (layer F.Cu) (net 20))
 (segment (start 100.24872 107.28452) (end 100.26572 107.26928) (width 0.2) (layer F.Cu) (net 20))
 (segment (start 100.095 106.085) (end 100.125 106.055) (width 0.2) (layer F.Cu) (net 20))
 (segment (start 100.095 106.635) (end 100.095 106.085) (width 0.2) (layer F.Cu) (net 20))
 (segment (start 98.0734 105.6215) (end 98.0734 104.7623) (width 0.2) (layer F.Cu) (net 20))
 (segment (start 98.0778 105.6259) (end 98.0734 105.6215) (width 0.2) (layer F.Cu) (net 20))
 (via (at 98.81616 106.74096) (size 0.8) (drill 0.4) (layers F.Cu B.Cu) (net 20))
 (segment (start 100.14712 105.41) (end 98.81616 106.74096) (width 0.508) (layer B.Cu) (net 20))
 (segment (start 98.07779 106.00259) (end 98.07779 105.6259) (width 0.2) (layer F.Cu) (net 20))
 (segment (start 98.81616 106.74096) (end 98.07779 106.00259) (width 0.2) (layer F.Cu) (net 20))
 (segment (start 99.998479 107.140959) (end 100.1268 107.26928) (width 0.2) (layer F.Cu) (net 20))
 (segment (start 99.216159 107.140959) (end 99.998479 107.140959) (width 0.2) (layer F.Cu) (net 20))
 (segment (start 98.81616 106.74096) (end 99.216159 107.140959) (width 0.2) (layer F.Cu) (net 20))
 (segment (start 106.68 105.41) (end 102.68712 105.39476) (width 0.508) (layer B.Cu) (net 20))
 (segment (start 102.68712 105.39476) (end 100.14712 105.41) (width 0.508) (layer B.Cu) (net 20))
 (segment (start 98.0734 104.7623) (end 98.0734 104.4408) (width 0.2) (layer F.Cu) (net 20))
 (segment (start 98.3292 104.185) (end 100.095 104.185) (width 0.2) (layer F.Cu) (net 20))
 (segment (start 98.0734 104.4408) (end 98.3292 104.185) (width 0.2) (layer F.Cu) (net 20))
 (segment (start 101.17836 103.886) (end 102.68712 105.39476) (width 0.508) (layer B.Cu) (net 20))
 (segment (start 101.1682 103.29164) (end 101.17836 103.886) (width 0.508) (layer B.Cu) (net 20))
 (segment (start 100.672292 103.31265) (end 100.4316 103.31265) (width 0.25) (layer B.Cu) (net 20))
 (segment (start 101.1682 103.29164) (end 100.693302 103.29164) (width 0.25) (layer B.Cu) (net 20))
 (segment (start 100.693302 103.29164) (end 100.672292 103.31265) (width 0.25) (layer B.Cu) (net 20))
 (segment (start 101.18348 103.27636) (end 101.96576 103.27636) (width 0.25) (layer B.Cu) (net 20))
 (segment (start 101.1682 103.29164) (end 101.18348 103.27636) (width 0.25) (layer B.Cu) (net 20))
 (via (at 101.17836 103.03256) (size 0.8) (drill 0.4) (layers F.Cu B.Cu) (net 20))
 (segment (start 100.955 104.185) (end 100.955 103.25592) (width 0.2) (layer F.Cu) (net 20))
 (segment (start 100.955 103.25592) (end 101.17836 103.03256) (width 0.2) (layer F.Cu) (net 20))
 (segment (start 100.5 106.055) (end 100.125 106.055) (width 0.2) (layer F.Cu) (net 20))
 (segment (start 100.600001 105.980001) (end 100.525002 106.055) (width 0.2) (layer F.Cu) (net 20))
 (segment (start 100.525002 106.055) (end 100.5 106.055) (width 0.2) (layer F.Cu) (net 20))
 (segment (start 100.525002 105.195) (end 100.600001 105.269999) (width 0.2) (layer F.Cu) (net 20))
 (segment (start 100.600001 105.269999) (end 100.600001 105.980001) (width 0.2) (layer F.Cu) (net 20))
 (segment (start 100.125 105.195) (end 100.525002 105.195) (width 0.2) (layer F.Cu) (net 20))
 (segment (start 101.98608 103.33876) (end 101.98608 103.10876) (width 0.2) (layer F.Cu) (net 21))
 (segment (start 101.98608 103.63892) (end 101.98608 103.33876) (width 0.2) (layer F.Cu) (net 21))
 (segment (start 101.815 103.81) (end 101.98608 103.63892) (width 0.2) (layer F.Cu) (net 21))
 (segment (start 101.815 104.185) (end 101.815 103.81) (width 0.2) (layer F.Cu) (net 21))
 (segment (start 100.4062 103.6912) (end 100.4062 103.35556) (width 0.2) (layer F.Cu) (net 22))
 (segment (start 100.4062 103.35556) (end 100.4062 103.15556) (width 0.2) (layer F.Cu) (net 22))
 (segment (start 100.525 103.81) (end 100.4062 103.6912) (width 0.2) (layer F.Cu) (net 22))
 (segment (start 100.525 104.185) (end 100.525 103.81) (width 0.2) (layer F.Cu) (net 22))
 (segment (start 102.635 74.015) (end 102.635 75.14) (width 0.42) (layer F.Cu) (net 14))
 (segment (start 103.005 73.645) (end 102.635 74.015) (width 0.42) (layer F.Cu) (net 14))
 (segment (start 116.205 73.645) (end 103.005 73.645) (width 0.42) (layer F.Cu) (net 14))
 (segment (start 101.985 74.015) (end 101.985 75.14) (width 0.42) (layer F.Cu) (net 14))
 (segment (start 102.355 73.645) (end 101.985 74.015) (width 0.42) (layer F.Cu) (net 14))
 (segment (start 103.005 73.645) (end 102.355 73.645) (width 0.42) (layer F.Cu) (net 14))
 (segment (start 100.035 76.435) (end 100.035 75.14) (width 0.42) (layer F.Cu) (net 13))
 (segment (start 116.205 77.145) (end 113.985 77.145) (width 0.42) (layer F.Cu) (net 13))
 (segment (start 104.7496 76.2) (end 104.0638 76.8858) (width 0.42) (layer F.Cu) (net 13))
 (segment (start 100.4858 76.8858) (end 100.035 76.435) (width 0.42) (layer F.Cu) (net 13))
 (segment (start 113.985 77.145) (end 113.04 76.2) (width 0.42) (layer F.Cu) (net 13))
 (segment (start 113.04 76.2) (end 104.7496 76.2) (width 0.42) (layer F.Cu) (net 13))
 (segment (start 104.0638 76.8858) (end 100.4858 76.8858) (width 0.42) (layer F.Cu) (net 13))
 (segment (start 99.385 76.435) (end 99.385 75.14) (width 0.42) (layer F.Cu) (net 13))
 (segment (start 99.8358 76.8858) (end 99.385 76.435) (width 0.42) (layer F.Cu) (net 13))
 (segment (start 100.4858 76.8858) (end 99.8358 76.8858) (width 0.42) (layer F.Cu) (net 13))
 (segment (start 88.9 72.39) (end 91.44 72.39) (width 0.25) (layer F.Cu) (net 25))
 (segment (start 90.102081 74.93) (end 91.44 74.93) (width 0.25) (layer F.Cu) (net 26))
 (segment (start 88.9 74.93) (end 90.102081 74.93) (width 0.25) (layer F.Cu) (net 26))
 (segment (start 90.102081 77.47) (end 91.44 77.47) (width 0.25) (layer F.Cu) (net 27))
 (segment (start 88.9 77.47) (end 90.102081 77.47) (width 0.25) (layer F.Cu) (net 27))
 (segment (start 91.44 82.55) (end 88.9 82.55) (width 0.25) (layer F.Cu) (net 28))
 (segment (start 90.102081 85.09) (end 91.44 85.09) (width 0.25) (layer F.Cu) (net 10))
 (segment (start 88.9 85.09) (end 90.102081 85.09) (width 0.25) (layer F.Cu) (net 10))
 (segment (start 90.102081 87.63) (end 91.44 87.63) (width 0.25) (layer F.Cu) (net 9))
 (segment (start 88.9 87.63) (end 90.102081 87.63) (width 0.25) (layer F.Cu) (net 9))
 (segment (start 90.102081 90.17) (end 91.44 90.17) (width 0.25) (layer F.Cu) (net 8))
 (segment (start 88.9 90.17) (end 90.102081 90.17) (width 0.25) (layer F.Cu) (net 8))
 (segment (start 88.9 92.71) (end 91.44 92.71) (width 0.25) (layer F.Cu) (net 6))
 (segment (start 88.9 95.25) (end 91.44 95.25) (width 0.25) (layer F.Cu) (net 4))
 (segment (start 90.102081 97.79) (end 91.44 97.79) (width 0.25) (layer F.Cu) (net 3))
 (segment (start 88.9 97.79) (end 90.102081 97.79) (width 0.25) (layer F.Cu) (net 3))
 (segment (start 90.102081 100.33) (end 91.44 100.33) (width 0.25) (layer F.Cu) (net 2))
 (segment (start 88.9 100.33) (end 90.102081 100.33) (width 0.25) (layer F.Cu) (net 2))
 (segment (start 88.9 102.87) (end 91.44 102.87) (width 0.25) (layer F.Cu) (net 29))
 (segment (start 90.237919 105.41) (end 88.9 105.41) (width 0.25) (layer F.Cu) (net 30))
 (segment (start 91.44 105.41) (end 90.237919 105.41) (width 0.25) (layer F.Cu) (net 30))
 (segment (start 90.102081 107.95) (end 91.44 107.95) (width 0.25) (layer F.Cu) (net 31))
 (segment (start 88.9 107.95) (end 90.102081 107.95) (width 0.25) (layer F.Cu) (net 31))
 (segment (start 108.017919 82.55) (end 106.68 82.55) (width 0.25) (layer F.Cu) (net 33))
 (segment (start 109.22 82.55) (end 108.017919 82.55) (width 0.25) (layer F.Cu) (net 33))
 (segment (start 108.017919 85.09) (end 106.68 85.09) (width 0.25) (layer F.Cu) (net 34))
 (segment (start 109.22 85.09) (end 108.017919 85.09) (width 0.25) (layer F.Cu) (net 34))
 (segment (start 108.017919 87.63) (end 106.68 87.63) (width 0.25) (layer F.Cu) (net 24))
 (segment (start 109.22 87.63) (end 108.017919 87.63) (width 0.25) (layer F.Cu) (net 24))
 (segment (start 100.1223 104.7623) (end 100.125 104.765) (width 0.2) (layer F.Cu) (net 24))
 (segment (start 98.5734 104.7623) (end 100.1223 104.7623) (width 0.2) (layer F.Cu) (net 24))
 (segment (start 108.017919 90.17) (end 106.68 90.17) (width 0.25) (layer F.Cu) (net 23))
 (segment (start 109.22 90.17) (end 108.017919 90.17) (width 0.25) (layer F.Cu) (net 23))
 (segment (start 100.1241 105.6259) (end 100.125 105.625) (width 0.2) (layer F.Cu) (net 23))
 (segment (start 98.5778 105.6259) (end 100.1241 105.6259) (width 0.2) (layer F.Cu) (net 23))
 (segment (start 109.22 92.71) (end 106.68 92.71) (width 0.25) (layer F.Cu) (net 35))
 (segment (start 108.017919 95.25) (end 106.68 95.25) (width 0.25) (layer F.Cu) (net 36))
 (segment (start 109.22 95.25) (end 108.017919 95.25) (width 0.25) (layer F.Cu) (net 36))
 (segment (start 108.017919 97.79) (end 106.68 97.79) (width 0.25) (layer F.Cu) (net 37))
 (segment (start 109.22 97.79) (end 108.017919 97.79) (width 0.25) (layer F.Cu) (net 37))
 (segment (start 108.017919 100.33) (end 106.68 100.33) (width 0.25) (layer F.Cu) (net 38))
 (segment (start 109.22 100.33) (end 108.017919 100.33) (width 0.25) (layer F.Cu) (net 38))
 (segment (start 108.017919 102.87) (end 106.68 102.87) (width 0.25) (layer F.Cu) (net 39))
 (segment (start 109.22 102.87) (end 108.017919 102.87) (width 0.25) (layer F.Cu) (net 39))
 (segment (start 108.017919 107.95) (end 106.68 107.95) (width 0.25) (layer F.Cu) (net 40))
 (segment (start 109.22 107.95) (end 108.017919 107.95) (width 0.25) (layer F.Cu) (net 40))
 (segment (start 109.22 77.47) (end 106.68 77.47) (width 0.25) (layer F.Cu) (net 32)))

